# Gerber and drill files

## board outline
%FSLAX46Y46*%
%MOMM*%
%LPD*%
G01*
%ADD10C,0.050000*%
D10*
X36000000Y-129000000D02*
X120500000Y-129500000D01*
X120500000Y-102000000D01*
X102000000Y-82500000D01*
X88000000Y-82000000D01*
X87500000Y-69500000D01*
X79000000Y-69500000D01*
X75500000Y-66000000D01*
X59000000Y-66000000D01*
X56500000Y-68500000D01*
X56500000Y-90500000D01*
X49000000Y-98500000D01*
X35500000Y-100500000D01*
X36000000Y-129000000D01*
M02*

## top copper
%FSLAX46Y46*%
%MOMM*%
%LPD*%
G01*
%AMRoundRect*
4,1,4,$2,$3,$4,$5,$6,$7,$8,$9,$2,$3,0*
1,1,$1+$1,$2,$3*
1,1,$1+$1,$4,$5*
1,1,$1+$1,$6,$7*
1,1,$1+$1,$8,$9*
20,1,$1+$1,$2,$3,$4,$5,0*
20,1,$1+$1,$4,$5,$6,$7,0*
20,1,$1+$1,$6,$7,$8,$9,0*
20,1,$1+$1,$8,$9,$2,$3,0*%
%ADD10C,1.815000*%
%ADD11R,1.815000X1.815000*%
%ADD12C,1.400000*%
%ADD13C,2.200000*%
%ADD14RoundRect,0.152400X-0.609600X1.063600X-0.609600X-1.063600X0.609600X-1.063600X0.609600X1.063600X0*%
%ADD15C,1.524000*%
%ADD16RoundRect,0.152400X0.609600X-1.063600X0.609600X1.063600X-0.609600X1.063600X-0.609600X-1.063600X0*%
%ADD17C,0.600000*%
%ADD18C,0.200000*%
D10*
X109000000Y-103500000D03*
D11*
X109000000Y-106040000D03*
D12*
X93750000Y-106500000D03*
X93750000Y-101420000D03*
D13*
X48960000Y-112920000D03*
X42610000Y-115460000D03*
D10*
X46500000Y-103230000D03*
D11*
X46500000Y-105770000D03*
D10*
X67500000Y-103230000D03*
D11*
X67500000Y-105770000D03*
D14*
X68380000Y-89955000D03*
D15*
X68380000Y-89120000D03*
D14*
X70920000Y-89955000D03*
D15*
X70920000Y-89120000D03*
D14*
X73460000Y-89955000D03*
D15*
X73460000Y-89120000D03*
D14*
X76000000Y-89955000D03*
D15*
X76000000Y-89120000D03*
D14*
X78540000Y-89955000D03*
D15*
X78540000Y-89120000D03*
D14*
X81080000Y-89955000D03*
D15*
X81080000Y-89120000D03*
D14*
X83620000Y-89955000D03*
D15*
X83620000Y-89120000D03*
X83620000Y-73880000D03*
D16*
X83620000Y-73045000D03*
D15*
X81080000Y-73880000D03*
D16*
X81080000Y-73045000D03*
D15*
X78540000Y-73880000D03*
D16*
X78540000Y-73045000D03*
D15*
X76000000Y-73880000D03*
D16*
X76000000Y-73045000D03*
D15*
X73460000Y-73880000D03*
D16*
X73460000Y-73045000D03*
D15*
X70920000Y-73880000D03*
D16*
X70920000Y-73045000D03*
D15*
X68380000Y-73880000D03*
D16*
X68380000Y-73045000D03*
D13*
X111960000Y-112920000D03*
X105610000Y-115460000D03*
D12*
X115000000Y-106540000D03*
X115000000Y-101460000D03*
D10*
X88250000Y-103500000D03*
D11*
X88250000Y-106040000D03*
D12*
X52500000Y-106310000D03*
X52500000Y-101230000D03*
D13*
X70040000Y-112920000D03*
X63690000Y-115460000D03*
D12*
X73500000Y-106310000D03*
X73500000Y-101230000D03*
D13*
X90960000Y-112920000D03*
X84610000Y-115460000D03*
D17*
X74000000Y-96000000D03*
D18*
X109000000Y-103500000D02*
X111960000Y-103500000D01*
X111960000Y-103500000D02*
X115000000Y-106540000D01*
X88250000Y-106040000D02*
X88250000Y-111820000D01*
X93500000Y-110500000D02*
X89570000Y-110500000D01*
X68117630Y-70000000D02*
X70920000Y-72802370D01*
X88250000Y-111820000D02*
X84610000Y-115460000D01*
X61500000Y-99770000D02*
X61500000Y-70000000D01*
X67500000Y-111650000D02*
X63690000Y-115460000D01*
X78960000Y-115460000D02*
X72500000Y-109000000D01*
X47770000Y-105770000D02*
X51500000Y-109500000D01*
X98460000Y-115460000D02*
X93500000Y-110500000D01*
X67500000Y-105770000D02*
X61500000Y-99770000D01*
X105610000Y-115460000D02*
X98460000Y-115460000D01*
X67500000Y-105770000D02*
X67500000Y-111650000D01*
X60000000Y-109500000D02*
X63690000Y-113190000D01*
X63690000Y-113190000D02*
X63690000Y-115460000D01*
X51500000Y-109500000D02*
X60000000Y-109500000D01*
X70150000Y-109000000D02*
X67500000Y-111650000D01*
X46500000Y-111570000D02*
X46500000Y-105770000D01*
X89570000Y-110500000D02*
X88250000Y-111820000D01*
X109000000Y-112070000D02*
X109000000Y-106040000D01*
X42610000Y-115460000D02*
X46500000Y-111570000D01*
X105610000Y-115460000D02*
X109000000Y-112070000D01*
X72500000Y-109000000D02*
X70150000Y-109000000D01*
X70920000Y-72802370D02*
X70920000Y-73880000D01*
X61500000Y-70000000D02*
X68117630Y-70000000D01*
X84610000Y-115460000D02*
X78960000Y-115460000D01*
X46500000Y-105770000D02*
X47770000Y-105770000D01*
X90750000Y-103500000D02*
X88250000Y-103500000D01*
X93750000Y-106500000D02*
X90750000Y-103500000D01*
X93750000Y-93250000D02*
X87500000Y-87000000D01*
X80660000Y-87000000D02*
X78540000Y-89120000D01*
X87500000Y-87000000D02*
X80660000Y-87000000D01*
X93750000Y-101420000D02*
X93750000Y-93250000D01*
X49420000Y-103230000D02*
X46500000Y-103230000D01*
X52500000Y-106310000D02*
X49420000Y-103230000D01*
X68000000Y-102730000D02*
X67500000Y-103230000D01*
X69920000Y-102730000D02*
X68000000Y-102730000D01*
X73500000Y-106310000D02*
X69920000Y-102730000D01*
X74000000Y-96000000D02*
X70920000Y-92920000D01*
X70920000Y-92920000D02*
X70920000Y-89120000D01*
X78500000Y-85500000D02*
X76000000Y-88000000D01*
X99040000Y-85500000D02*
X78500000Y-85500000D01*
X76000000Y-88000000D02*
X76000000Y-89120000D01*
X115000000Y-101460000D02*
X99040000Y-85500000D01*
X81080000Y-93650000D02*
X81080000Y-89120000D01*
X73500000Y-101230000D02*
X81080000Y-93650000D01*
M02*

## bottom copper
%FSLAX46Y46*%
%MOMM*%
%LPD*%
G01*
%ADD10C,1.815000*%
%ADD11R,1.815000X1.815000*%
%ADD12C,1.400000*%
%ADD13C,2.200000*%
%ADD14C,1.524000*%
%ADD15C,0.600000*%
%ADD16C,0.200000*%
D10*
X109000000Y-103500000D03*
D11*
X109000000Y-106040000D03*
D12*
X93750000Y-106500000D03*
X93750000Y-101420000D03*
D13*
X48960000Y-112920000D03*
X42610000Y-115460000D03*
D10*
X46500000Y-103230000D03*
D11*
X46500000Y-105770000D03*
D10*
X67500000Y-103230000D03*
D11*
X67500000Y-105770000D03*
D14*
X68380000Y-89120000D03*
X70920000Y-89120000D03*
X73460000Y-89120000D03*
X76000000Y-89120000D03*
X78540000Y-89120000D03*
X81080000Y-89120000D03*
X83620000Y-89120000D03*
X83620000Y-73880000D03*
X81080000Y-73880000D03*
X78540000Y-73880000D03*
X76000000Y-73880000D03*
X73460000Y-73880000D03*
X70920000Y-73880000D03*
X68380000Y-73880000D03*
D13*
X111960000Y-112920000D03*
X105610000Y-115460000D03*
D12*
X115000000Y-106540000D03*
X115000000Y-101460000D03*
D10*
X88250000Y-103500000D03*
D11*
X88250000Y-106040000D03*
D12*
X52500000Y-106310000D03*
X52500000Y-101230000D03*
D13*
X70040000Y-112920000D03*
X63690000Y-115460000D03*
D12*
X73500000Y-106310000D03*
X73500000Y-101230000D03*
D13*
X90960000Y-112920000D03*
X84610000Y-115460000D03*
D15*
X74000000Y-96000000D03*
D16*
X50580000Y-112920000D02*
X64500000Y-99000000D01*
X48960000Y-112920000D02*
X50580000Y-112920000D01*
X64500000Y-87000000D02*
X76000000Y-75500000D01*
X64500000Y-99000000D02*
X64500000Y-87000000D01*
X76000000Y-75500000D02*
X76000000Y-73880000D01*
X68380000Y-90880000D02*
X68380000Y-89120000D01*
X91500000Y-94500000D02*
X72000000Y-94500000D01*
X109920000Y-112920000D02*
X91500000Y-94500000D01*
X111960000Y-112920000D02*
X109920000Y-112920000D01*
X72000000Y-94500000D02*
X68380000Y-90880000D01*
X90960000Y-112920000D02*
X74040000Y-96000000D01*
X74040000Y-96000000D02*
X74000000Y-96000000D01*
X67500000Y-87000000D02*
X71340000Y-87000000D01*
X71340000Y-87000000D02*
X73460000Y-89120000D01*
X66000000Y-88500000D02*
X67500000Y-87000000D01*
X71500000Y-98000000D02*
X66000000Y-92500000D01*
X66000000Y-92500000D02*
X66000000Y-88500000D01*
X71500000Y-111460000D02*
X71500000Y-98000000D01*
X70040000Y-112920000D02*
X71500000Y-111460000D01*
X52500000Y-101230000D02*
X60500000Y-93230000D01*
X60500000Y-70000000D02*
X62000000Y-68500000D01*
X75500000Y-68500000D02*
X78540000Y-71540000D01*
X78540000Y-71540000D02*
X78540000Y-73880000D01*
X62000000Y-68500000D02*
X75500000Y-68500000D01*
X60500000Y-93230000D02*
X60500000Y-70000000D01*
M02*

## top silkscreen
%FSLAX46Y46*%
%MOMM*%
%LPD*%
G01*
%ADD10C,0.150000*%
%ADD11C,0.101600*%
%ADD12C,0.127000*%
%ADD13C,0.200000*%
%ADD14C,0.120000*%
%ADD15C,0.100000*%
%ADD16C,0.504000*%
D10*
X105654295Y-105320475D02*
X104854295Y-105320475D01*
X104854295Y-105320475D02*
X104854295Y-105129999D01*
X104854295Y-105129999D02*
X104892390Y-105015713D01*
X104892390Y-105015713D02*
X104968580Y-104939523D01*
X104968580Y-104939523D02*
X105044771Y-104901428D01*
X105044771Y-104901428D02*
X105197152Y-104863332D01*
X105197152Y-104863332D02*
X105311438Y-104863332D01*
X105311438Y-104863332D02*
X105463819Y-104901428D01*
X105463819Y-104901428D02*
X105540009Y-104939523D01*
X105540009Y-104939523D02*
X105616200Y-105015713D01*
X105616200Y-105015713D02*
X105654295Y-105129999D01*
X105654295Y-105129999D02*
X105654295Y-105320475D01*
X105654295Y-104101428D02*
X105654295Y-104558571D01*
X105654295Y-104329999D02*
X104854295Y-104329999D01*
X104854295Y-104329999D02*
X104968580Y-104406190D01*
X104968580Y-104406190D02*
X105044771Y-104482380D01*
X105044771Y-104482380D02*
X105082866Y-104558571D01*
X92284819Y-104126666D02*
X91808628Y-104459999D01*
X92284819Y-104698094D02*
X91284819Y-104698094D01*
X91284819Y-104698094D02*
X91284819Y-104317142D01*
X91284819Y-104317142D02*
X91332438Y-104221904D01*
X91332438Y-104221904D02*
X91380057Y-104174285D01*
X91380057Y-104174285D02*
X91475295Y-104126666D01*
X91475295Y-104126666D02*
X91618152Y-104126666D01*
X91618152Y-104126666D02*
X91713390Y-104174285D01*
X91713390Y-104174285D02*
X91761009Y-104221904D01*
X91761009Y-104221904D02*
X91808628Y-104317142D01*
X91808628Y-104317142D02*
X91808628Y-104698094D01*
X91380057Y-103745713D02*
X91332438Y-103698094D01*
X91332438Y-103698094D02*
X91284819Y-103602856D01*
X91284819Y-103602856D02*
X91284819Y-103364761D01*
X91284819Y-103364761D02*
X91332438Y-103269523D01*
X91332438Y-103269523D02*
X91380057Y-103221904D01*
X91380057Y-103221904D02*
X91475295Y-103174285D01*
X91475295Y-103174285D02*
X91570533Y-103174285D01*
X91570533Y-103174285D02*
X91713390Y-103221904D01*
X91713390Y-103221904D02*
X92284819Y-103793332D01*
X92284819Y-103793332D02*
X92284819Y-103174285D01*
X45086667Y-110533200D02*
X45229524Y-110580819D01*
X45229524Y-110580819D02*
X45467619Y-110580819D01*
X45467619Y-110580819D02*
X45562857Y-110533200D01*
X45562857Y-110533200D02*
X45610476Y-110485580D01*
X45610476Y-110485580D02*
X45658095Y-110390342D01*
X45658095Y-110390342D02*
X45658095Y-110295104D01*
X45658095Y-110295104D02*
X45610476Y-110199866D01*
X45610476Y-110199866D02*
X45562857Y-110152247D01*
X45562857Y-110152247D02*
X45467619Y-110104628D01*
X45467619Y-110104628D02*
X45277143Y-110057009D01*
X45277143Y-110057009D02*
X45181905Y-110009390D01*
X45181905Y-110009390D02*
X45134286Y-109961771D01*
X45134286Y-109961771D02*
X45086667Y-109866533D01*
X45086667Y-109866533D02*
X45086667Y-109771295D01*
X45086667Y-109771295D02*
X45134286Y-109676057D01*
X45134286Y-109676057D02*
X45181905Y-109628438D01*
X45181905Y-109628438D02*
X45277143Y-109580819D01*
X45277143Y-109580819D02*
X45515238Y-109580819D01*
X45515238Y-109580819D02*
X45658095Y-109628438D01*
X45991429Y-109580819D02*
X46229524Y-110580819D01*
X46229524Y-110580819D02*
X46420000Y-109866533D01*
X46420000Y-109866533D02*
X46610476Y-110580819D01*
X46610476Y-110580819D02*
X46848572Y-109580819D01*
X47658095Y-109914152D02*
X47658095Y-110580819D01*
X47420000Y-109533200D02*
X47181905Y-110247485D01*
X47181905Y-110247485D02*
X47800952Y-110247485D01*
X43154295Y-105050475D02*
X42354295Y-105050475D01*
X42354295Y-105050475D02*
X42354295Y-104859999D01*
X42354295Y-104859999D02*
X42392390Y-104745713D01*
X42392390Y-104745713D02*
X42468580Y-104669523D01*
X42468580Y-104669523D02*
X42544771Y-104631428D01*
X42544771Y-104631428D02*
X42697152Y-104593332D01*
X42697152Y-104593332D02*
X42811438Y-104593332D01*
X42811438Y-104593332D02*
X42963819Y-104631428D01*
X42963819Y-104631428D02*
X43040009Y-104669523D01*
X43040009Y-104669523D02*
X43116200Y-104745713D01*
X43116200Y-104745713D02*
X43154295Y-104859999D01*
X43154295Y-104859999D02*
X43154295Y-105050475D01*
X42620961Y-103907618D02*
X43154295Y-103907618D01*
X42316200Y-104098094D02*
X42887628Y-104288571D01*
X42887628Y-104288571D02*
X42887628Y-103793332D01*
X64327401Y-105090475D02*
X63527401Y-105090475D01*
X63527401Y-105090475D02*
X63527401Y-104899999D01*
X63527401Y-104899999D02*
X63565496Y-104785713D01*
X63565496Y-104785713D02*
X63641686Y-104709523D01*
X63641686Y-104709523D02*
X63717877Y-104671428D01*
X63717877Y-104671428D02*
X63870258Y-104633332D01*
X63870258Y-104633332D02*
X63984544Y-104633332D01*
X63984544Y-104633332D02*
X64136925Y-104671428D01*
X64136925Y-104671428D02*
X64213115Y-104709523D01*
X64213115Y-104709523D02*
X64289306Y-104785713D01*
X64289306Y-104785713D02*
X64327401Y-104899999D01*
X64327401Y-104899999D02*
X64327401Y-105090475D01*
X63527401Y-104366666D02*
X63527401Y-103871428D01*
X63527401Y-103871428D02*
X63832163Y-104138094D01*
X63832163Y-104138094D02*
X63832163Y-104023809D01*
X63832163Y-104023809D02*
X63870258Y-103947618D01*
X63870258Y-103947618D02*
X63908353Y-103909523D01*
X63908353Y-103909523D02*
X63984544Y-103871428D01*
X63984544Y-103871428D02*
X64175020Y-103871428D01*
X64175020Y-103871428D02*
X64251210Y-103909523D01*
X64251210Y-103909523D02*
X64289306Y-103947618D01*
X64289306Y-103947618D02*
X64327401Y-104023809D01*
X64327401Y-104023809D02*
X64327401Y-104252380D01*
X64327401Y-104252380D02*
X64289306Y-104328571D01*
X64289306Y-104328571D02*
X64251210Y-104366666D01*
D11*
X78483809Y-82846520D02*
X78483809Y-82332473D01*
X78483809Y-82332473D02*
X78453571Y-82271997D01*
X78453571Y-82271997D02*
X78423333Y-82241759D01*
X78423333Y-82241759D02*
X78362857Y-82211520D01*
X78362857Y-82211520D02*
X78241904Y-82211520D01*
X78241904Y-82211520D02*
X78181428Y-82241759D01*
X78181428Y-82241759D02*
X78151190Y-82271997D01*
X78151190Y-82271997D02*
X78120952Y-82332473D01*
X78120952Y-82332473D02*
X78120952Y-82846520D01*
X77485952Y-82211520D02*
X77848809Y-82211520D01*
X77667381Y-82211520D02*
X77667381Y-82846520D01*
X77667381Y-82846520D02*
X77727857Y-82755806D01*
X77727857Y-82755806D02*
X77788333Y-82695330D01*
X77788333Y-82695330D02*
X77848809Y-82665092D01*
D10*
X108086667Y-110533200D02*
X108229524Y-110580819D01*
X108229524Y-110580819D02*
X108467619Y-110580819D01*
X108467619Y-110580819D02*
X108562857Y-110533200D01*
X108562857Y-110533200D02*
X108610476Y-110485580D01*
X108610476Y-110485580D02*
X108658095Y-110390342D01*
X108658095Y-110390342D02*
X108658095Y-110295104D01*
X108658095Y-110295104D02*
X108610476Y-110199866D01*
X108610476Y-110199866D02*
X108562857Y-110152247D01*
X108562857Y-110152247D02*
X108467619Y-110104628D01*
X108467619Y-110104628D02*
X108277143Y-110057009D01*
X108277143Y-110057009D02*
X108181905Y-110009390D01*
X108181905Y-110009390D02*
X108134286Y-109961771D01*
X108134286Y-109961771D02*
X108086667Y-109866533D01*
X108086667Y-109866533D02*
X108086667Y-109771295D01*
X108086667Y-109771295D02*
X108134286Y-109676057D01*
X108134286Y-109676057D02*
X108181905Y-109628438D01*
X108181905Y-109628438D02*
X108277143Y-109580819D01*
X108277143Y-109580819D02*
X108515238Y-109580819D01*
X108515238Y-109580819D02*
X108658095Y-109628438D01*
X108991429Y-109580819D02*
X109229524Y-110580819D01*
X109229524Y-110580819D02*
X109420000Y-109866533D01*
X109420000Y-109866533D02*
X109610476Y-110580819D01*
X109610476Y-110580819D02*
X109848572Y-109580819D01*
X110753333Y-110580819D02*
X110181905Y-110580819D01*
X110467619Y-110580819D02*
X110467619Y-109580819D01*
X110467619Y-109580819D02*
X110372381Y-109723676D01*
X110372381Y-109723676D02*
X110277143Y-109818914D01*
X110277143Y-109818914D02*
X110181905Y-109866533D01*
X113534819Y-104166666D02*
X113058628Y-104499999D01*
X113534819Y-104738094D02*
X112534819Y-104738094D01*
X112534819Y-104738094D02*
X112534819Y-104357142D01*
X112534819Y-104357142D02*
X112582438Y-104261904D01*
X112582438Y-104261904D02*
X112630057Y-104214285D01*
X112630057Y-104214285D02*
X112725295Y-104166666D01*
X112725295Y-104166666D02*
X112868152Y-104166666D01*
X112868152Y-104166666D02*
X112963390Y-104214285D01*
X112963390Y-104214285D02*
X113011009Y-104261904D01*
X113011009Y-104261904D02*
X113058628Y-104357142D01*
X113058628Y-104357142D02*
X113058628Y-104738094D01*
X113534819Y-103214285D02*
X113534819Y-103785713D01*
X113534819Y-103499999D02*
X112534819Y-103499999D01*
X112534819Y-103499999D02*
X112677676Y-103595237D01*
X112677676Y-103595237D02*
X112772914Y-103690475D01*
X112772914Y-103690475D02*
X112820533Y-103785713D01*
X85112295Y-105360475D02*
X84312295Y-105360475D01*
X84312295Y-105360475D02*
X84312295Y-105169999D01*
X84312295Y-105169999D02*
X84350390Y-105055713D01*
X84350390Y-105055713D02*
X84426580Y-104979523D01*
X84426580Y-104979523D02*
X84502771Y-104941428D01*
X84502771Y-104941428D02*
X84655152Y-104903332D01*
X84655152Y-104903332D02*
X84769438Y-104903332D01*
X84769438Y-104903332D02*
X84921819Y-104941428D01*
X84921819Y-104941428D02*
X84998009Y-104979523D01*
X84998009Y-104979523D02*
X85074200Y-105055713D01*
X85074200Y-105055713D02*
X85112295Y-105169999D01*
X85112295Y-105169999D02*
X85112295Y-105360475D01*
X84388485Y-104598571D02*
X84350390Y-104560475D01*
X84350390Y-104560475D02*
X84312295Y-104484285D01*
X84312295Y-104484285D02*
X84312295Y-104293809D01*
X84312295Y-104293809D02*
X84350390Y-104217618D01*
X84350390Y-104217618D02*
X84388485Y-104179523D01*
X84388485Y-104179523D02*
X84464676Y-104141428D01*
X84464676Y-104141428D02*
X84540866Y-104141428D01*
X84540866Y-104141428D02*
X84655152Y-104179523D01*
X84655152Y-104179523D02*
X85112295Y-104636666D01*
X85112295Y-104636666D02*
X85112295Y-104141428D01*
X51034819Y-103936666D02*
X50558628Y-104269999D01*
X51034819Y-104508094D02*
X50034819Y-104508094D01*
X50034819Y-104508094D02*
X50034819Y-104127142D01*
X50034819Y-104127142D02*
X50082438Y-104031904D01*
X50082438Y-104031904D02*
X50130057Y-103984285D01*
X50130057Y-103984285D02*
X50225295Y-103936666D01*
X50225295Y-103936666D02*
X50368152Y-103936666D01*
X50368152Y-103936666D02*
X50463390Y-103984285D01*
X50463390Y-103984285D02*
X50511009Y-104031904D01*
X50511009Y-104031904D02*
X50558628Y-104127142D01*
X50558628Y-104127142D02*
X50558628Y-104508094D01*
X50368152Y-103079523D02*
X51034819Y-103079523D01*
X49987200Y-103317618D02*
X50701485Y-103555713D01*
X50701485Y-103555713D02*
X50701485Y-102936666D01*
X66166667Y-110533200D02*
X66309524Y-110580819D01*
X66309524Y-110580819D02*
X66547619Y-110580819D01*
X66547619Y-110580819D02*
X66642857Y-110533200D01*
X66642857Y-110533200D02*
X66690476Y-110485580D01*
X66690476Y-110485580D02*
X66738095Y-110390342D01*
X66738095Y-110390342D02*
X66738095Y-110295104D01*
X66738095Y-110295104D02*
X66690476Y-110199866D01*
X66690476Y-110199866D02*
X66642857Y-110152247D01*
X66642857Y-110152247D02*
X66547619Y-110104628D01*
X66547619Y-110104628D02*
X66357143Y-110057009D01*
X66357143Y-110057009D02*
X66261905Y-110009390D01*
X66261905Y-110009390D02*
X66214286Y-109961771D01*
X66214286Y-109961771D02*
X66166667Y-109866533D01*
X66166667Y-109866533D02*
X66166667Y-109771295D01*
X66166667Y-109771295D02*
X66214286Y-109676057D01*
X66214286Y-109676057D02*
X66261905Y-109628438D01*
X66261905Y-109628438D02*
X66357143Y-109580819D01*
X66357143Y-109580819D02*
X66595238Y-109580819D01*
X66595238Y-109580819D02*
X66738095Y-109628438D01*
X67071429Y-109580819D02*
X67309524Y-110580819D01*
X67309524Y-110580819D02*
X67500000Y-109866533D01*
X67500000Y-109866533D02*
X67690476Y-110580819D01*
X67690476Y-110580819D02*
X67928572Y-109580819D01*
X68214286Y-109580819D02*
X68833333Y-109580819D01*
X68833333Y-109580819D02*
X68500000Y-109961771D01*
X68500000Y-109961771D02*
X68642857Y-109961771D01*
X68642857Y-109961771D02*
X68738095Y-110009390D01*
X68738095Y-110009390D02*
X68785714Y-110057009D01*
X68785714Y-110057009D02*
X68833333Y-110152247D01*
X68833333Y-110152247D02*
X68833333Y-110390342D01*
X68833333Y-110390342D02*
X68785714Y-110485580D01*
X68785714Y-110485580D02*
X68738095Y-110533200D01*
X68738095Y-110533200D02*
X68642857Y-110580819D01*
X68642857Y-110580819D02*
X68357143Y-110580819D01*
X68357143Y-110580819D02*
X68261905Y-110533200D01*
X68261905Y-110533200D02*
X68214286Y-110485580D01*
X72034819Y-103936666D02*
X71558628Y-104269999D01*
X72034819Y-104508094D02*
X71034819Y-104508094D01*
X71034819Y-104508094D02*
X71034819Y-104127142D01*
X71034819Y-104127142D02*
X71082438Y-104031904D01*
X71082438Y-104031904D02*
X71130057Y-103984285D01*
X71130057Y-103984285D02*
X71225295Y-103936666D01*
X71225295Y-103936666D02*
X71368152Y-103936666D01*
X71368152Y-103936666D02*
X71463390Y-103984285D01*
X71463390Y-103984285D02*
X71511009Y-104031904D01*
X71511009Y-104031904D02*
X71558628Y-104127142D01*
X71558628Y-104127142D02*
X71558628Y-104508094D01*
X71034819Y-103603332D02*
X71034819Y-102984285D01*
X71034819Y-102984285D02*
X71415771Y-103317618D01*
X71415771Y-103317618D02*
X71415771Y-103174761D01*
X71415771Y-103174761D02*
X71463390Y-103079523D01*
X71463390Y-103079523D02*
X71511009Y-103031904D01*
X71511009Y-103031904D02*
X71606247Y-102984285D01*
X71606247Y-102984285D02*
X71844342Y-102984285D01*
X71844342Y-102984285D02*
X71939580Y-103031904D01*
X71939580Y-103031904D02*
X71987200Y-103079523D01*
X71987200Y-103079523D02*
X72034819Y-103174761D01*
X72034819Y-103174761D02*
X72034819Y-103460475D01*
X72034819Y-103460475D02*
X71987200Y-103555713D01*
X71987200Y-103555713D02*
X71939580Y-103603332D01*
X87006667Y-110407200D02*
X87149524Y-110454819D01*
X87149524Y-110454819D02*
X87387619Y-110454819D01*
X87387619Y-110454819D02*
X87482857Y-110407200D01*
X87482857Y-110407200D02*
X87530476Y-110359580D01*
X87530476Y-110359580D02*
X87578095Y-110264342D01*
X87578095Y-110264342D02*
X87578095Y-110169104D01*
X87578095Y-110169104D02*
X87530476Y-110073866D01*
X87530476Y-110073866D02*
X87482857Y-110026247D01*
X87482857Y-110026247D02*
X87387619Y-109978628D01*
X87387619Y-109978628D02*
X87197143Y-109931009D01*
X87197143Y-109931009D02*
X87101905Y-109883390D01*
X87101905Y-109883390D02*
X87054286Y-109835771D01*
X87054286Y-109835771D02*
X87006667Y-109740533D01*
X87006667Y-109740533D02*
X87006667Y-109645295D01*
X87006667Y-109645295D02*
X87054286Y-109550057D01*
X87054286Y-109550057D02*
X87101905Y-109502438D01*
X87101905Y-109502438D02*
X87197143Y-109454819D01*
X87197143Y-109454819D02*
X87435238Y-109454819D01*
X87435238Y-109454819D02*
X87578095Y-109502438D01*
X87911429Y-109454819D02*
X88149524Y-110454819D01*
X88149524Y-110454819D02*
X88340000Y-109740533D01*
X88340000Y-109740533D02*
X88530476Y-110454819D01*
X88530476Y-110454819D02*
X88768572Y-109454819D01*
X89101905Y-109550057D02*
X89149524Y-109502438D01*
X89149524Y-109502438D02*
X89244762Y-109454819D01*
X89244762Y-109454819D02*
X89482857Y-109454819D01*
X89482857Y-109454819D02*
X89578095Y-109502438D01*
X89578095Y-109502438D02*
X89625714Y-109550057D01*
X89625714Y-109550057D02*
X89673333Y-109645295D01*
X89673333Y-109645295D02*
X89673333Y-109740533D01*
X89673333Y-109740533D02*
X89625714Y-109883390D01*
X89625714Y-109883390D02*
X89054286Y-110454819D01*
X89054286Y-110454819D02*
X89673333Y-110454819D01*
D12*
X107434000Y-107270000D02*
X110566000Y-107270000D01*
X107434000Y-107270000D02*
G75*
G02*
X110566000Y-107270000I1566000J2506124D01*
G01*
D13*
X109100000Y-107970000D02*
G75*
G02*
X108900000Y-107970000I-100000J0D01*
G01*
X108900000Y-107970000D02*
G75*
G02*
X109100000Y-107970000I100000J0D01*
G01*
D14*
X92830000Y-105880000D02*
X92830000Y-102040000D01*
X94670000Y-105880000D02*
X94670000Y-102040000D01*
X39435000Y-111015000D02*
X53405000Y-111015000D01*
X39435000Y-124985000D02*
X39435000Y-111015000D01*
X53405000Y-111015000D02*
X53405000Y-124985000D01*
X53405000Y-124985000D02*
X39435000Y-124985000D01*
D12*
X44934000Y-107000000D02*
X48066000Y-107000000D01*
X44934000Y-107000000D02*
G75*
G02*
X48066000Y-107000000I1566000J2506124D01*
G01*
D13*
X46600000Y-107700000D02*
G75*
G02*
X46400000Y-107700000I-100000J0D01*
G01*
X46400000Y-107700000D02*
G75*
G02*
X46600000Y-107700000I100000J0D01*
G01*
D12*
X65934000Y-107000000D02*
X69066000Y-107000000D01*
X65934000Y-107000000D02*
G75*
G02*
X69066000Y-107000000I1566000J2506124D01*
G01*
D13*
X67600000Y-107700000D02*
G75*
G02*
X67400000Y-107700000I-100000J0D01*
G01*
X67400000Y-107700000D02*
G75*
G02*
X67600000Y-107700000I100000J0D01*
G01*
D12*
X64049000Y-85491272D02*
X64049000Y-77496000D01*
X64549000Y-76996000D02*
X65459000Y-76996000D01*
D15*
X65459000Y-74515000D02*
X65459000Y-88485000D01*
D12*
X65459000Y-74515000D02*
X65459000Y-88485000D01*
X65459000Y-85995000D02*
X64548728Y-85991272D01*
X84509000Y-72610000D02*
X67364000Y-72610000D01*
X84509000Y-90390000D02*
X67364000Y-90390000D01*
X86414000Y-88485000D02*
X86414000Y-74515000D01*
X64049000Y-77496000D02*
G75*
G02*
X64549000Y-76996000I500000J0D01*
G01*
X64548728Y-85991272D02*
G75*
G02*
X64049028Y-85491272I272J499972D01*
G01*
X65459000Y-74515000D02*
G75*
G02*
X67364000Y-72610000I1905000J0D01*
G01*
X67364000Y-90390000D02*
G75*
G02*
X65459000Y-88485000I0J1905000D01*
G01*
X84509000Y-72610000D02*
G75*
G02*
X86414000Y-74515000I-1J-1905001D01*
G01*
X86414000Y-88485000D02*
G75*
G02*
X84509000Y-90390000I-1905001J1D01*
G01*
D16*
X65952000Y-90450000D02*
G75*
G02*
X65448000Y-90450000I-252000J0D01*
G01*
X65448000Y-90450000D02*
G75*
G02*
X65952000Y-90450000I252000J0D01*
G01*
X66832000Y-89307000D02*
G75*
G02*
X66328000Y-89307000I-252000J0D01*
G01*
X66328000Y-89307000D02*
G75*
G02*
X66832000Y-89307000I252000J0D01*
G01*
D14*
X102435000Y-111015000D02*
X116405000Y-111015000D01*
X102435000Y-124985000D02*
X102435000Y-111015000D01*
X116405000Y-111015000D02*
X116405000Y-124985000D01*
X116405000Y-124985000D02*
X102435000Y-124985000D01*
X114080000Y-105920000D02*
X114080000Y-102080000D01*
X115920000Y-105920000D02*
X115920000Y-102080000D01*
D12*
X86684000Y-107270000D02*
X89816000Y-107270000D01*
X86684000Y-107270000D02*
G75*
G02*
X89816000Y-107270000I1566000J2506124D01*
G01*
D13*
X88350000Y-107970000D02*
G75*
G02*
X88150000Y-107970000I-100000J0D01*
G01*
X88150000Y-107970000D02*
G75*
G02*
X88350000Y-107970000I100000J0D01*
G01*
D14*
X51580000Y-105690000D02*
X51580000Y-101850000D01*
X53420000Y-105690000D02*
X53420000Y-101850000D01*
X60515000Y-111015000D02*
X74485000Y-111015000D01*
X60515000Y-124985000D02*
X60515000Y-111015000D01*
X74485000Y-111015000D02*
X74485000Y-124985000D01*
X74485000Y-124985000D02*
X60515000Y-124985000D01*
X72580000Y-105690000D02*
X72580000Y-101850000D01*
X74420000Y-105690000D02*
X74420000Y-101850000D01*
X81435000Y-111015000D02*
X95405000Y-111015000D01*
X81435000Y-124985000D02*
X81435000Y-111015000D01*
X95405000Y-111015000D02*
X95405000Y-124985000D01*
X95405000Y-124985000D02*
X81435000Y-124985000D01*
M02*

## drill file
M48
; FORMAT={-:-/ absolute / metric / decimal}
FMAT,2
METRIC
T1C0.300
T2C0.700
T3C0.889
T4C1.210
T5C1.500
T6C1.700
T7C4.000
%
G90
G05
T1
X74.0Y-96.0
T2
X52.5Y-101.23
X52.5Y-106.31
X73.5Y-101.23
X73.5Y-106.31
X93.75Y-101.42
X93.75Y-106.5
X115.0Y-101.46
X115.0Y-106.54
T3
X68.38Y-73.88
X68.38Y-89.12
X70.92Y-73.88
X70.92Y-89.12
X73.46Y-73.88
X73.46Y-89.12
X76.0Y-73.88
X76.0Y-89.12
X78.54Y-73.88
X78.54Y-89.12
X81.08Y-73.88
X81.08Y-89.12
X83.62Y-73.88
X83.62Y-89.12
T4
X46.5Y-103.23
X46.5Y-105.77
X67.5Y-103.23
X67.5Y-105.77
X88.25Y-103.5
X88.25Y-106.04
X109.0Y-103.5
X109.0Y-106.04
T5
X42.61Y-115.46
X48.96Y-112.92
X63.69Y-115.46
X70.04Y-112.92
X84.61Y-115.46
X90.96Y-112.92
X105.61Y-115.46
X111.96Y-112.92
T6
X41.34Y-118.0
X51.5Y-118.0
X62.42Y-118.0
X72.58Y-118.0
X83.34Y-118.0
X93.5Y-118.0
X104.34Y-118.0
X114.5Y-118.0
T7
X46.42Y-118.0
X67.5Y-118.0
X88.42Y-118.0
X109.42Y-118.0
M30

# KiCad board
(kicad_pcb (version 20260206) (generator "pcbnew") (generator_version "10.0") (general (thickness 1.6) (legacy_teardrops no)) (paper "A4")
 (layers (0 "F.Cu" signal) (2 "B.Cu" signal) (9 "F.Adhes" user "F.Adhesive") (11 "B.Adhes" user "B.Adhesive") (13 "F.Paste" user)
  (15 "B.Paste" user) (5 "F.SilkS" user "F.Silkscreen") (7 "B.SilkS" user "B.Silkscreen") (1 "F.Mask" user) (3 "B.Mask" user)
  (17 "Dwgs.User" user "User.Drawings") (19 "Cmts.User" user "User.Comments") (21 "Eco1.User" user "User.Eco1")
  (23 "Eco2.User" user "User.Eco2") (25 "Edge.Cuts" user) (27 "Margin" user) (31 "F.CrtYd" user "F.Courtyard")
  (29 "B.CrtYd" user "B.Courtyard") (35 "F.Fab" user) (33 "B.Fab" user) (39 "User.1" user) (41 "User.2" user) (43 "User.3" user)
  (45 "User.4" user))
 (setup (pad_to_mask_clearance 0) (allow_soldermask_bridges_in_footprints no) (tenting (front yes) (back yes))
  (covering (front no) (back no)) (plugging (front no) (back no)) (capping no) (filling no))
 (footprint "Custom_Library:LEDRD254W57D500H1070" (layer "F.Cu") (at 109 104.77 90)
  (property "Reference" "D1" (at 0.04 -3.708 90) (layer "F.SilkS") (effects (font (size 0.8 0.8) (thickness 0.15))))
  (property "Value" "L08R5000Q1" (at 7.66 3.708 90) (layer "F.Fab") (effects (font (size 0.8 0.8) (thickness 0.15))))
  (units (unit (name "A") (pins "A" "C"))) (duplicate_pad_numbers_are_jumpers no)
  (fp_line (start -2.5 -1.566) (end -2.5 1.566) (stroke (width 0.127) (type solid)) (layer "F.SilkS"))
  (fp_arc (start -2.5 -1.566) (mid 2.961291 0) (end -2.5 1.566) (stroke (width 0.127) (type solid)) (layer "F.SilkS"))
  (fp_circle (center -3.2 0) (end -3.1 0) (stroke (width 0.2) (type solid)) (fill no) (layer "F.SilkS"))
  (pad "A" thru_hole circle (at 1.27 0 90) (size 1.815 1.815) (drill 1.21) (layers "*.Cu" "*.Mask") (remove_unused_layers no)
   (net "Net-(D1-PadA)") (solder_mask_margin 0.102))
  (pad "C" thru_hole rect (at -1.27 0 90) (size 1.815 1.815) (drill 1.21) (layers "*.Cu" "*.Mask") (remove_unused_layers no) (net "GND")
   (solder_mask_margin 0.102)))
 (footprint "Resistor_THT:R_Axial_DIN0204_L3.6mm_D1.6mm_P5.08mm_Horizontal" (layer "F.Cu") (at 93.75 106.5 90)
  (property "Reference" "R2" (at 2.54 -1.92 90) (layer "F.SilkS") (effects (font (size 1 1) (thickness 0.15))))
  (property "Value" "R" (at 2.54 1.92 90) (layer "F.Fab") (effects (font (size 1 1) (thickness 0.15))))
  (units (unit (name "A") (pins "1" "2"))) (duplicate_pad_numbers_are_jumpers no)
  (fp_line (start 0.62 -0.92) (end 4.46 -0.92) (stroke (width 0.12) (type solid)) (layer "F.SilkS"))
  (fp_line (start 0.62 0.92) (end 4.46 0.92) (stroke (width 0.12) (type solid)) (layer "F.SilkS"))
  (pad "1" thru_hole circle (at 0 0 90) (size 1.4 1.4) (drill 0.7) (layers "*.Cu" "*.Mask") (remove_unused_layers no) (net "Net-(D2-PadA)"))
  (pad "2" thru_hole circle (at 5.08 0 90) (size 1.4 1.4) (drill 0.7) (layers "*.Cu" "*.Mask") (remove_unused_layers no) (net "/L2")))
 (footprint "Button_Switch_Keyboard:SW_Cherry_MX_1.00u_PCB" (layer "F.Cu") (at 48.96 112.92)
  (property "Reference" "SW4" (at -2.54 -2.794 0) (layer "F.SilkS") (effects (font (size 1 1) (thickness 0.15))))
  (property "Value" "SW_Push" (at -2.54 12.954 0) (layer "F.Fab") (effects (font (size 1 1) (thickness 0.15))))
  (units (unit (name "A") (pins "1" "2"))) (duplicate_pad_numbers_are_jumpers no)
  (fp_line (start -9.525 -1.905) (end 4.445 -1.905) (stroke (width 0.12) (type solid)) (layer "F.SilkS"))
  (fp_line (start -9.525 12.065) (end -9.525 -1.905) (stroke (width 0.12) (type solid)) (layer "F.SilkS"))
  (fp_line (start 4.445 -1.905) (end 4.445 12.065) (stroke (width 0.12) (type solid)) (layer "F.SilkS"))
  (fp_line (start 4.445 12.065) (end -9.525 12.065) (stroke (width 0.12) (type solid)) (layer "F.SilkS"))
  (pad "" np_thru_hole circle (at -7.62 5.08) (size 1.7 1.7) (drill 1.7) (layers "*.Cu" "*.Mask"))
  (pad "" np_thru_hole circle (at -2.54 5.08) (size 4 4) (drill 4) (layers "*.Cu" "*.Mask"))
  (pad "" np_thru_hole circle (at 2.54 5.08) (size 1.7 1.7) (drill 1.7) (layers "*.Cu" "*.Mask"))
  (pad "1" thru_hole circle (at 0 0) (size 2.2 2.2) (drill 1.5) (layers "*.Cu" "*.Mask") (remove_unused_layers no) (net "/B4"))
  (pad "2" thru_hole circle (at -6.35 2.54) (size 2.2 2.2) (drill 1.5) (layers "*.Cu" "*.Mask") (remove_unused_layers no) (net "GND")))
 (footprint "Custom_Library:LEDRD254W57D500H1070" (layer "F.Cu") (at 46.5 104.5 90)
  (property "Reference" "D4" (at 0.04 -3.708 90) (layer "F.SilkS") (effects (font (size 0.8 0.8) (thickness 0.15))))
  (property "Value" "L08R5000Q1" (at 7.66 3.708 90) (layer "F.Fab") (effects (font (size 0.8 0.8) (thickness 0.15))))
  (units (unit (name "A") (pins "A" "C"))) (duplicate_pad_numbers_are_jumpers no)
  (fp_line (start -2.5 -1.566) (end -2.5 1.566) (stroke (width 0.127) (type solid)) (layer "F.SilkS"))
  (fp_arc (start -2.5 -1.566) (mid 2.961291 0) (end -2.5 1.566) (stroke (width 0.127) (type solid)) (layer "F.SilkS"))
  (fp_circle (center -3.2 0) (end -3.1 0) (stroke (width 0.2) (type solid)) (fill no) (layer "F.SilkS"))
  (pad "A" thru_hole circle (at 1.27 0 90) (size 1.815 1.815) (drill 1.21) (layers "*.Cu" "*.Mask") (remove_unused_layers no)
   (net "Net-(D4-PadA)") (solder_mask_margin 0.102))
  (pad "C" thru_hole rect (at -1.27 0 90) (size 1.815 1.815) (drill 1.21) (layers "*.Cu" "*.Mask") (remove_unused_layers no) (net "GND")
   (solder_mask_margin 0.102)))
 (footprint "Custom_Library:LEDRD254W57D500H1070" (layer "F.Cu") (at 67.5 104.5 90)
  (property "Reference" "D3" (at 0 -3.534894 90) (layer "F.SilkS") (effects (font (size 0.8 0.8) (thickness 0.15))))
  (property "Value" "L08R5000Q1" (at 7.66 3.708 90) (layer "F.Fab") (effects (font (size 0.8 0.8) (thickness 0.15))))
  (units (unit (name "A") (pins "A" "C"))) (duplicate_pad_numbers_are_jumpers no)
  (fp_line (start -2.5 -1.566) (end -2.5 1.566) (stroke (width 0.127) (type solid)) (layer "F.SilkS"))
  (fp_arc (start -2.5 -1.566) (mid 2.961291 0) (end -2.5 1.566) (stroke (width 0.127) (type solid)) (layer "F.SilkS"))
  (fp_circle (center -3.2 0) (end -3.1 0) (stroke (width 0.2) (type solid)) (fill no) (layer "F.SilkS"))
  (pad "A" thru_hole circle (at 1.27 0 90) (size 1.815 1.815) (drill 1.21) (layers "*.Cu" "*.Mask") (remove_unused_layers no)
   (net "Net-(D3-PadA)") (solder_mask_margin 0.102))
  (pad "C" thru_hole rect (at -1.27 0 90) (size 1.815 1.815) (drill 1.21) (layers "*.Cu" "*.Mask") (remove_unused_layers no) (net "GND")
   (solder_mask_margin 0.102)))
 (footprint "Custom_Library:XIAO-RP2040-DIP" (layer "F.Cu") (at 76 81.5 180)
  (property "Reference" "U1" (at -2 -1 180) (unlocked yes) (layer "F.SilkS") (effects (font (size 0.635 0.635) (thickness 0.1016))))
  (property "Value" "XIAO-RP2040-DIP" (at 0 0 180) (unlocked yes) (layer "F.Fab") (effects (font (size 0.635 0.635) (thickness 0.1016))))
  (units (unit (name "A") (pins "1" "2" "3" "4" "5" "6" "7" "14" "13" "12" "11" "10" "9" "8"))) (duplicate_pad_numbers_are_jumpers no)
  (fp_line (start 11.951 -3.991272) (end 11.951 4.004) (stroke (width 0.127) (type solid)) (layer "F.SilkS"))
  (fp_line (start 11.451 4.504) (end 10.541 4.504) (stroke (width 0.127) (type solid)) (layer "F.SilkS"))
  (fp_line (start 10.541 6.985) (end 10.541 -6.985) (stroke (width 0.1) (type solid)) (layer "F.SilkS"))
  (fp_line (start 10.541 6.985) (end 10.541 -6.985) (stroke (width 0.127) (type solid)) (layer "F.SilkS"))
  (fp_line (start 10.541 -4.495) (end 11.451272 -4.491272) (stroke (width 0.127) (type solid)) (layer "F.SilkS"))
  (fp_line (start -8.509 8.89) (end 8.636 8.89) (stroke (width 0.127) (type solid)) (layer "F.SilkS"))
  (fp_line (start -8.509 -8.89) (end 8.636 -8.89) (stroke (width 0.127) (type solid)) (layer "F.SilkS"))
  (fp_line (start -10.414 -6.985) (end -10.414 6.985) (stroke (width 0.127) (type solid)) (layer "F.SilkS"))
  (fp_arc (start 11.951 4.004) (mid 11.804553 4.357553) (end 11.451 4.504) (stroke (width 0.127) (type default)) (layer "F.SilkS"))
  (fp_arc (start 11.451272 -4.491272) (mid 11.804644 -4.344724) (end 11.951 -3.991272) (stroke (width 0.127) (type default))
   (layer "F.SilkS"))
  (fp_arc (start 10.541 6.985) (mid 9.983038 8.332038) (end 8.636 8.89) (stroke (width 0.127) (type solid)) (layer "F.SilkS"))
  (fp_arc (start 8.636 -8.89) (mid 9.983038 -8.332038) (end 10.541 -6.985) (stroke (width 0.127) (type solid)) (layer "F.SilkS"))
  (fp_arc (start -8.509 8.89) (mid -9.856038 8.332038) (end -10.414 6.985) (stroke (width 0.127) (type solid)) (layer "F.SilkS"))
  (fp_arc (start -10.414 -6.985) (mid -9.856038 -8.332038) (end -8.509 -8.89) (stroke (width 0.127) (type solid)) (layer "F.SilkS"))
  (fp_circle (center 10.3 -8.95) (end 10.554 -8.95) (stroke (width 0.5) (type solid)) (fill yes) (layer "F.SilkS"))
  (fp_circle (center 9.42 -7.807) (end 9.674 -7.807) (stroke (width 0.5) (type solid)) (fill yes) (layer "F.SilkS"))
  (pad "1" smd roundrect (at 7.62 -8.455 270) (size 2.432 1.524) (layers "F.Cu" "F.Mask") (roundrect_rratio 0.1) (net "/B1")
   (thermal_bridge_angle 45))
  (pad "1" thru_hole circle (at 7.62 -7.62 270) (size 1.524 1.524) (drill 0.889) (layers "*.Cu" "*.Mask") (remove_unused_layers no)
   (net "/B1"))
  (pad "2" smd roundrect (at 5.08 -8.455 270) (size 2.432 1.524) (layers "F.Cu" "F.Mask") (roundrect_rratio 0.1) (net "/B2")
   (thermal_bridge_angle 45))
  (pad "2" thru_hole circle (at 5.08 -7.62 270) (size 1.524 1.524) (drill 0.889) (layers "*.Cu" "*.Mask") (remove_unused_layers no)
   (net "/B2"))
  (pad "3" smd roundrect (at 2.54 -8.455 270) (size 2.432 1.524) (layers "F.Cu" "F.Mask") (roundrect_rratio 0.1) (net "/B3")
   (thermal_bridge_angle 45))
  (pad "3" thru_hole circle (at 2.54 -7.62 270) (size 1.524 1.524) (drill 0.889) (layers "*.Cu" "*.Mask") (remove_unused_layers no)
   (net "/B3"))
  (pad "4" smd roundrect (at 0 -8.455 270) (size 2.432 1.524) (layers "F.Cu" "F.Mask") (roundrect_rratio 0.1) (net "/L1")
   (thermal_bridge_angle 45))
  (pad "4" thru_hole circle (at 0 -7.62 270) (size 1.524 1.524) (drill 0.889) (layers "*.Cu" "*.Mask") (remove_unused_layers no) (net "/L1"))
  (pad "5" smd roundrect (at -2.54 -8.455 270) (size 2.432 1.524) (layers "F.Cu" "F.Mask") (roundrect_rratio 0.1) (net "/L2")
   (thermal_bridge_angle 45))
  (pad "5" thru_hole circle (at -2.54 -7.62 270) (size 1.524 1.524) (drill 0.889) (layers "*.Cu" "*.Mask") (remove_unused_layers no)
   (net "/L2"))
  (pad "6" smd roundrect (at -5.08 -8.455 270) (size 2.432 1.524) (layers "F.Cu" "F.Mask") (roundrect_rratio 0.1) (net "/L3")
   (thermal_bridge_angle 45))
  (pad "6" thru_hole circle (at -5.08 -7.62 270) (size 1.524 1.524) (drill 0.889) (layers "*.Cu" "*.Mask") (remove_unused_layers no)
   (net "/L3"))
  (pad "7" smd roundrect (at -7.62 -8.455 270) (size 2.432 1.524) (layers "F.Cu" "F.Mask") (roundrect_rratio 0.1)
   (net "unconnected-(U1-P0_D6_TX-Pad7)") (thermal_bridge_angle 45))
  (pad "7" thru_hole circle (at -7.62 -7.62 270) (size 1.524 1.524) (drill 0.889) (layers "*.Cu" "*.Mask") (remove_unused_layers no)
   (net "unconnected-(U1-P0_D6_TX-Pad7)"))
  (pad "8" thru_hole circle (at -7.62 7.62 90) (size 1.524 1.524) (drill 0.889) (layers "*.Cu" "*.Mask") (remove_unused_layers no)
   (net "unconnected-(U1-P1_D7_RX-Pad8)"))
  (pad "8" smd roundrect (at -7.62 8.455 90) (size 2.432 1.524) (layers "F.Cu" "F.Mask") (roundrect_rratio 0.1)
   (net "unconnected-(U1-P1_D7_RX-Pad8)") (thermal_bridge_angle 45))
  (pad "9" thru_hole circle (at -5.08 7.62 90) (size 1.524 1.524) (drill 0.889) (layers "*.Cu" "*.Mask") (remove_unused_layers no)
   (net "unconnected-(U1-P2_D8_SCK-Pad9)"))
  (pad "9" smd roundrect (at -5.08 8.455 90) (size 2.432 1.524) (layers "F.Cu" "F.Mask") (roundrect_rratio 0.1)
   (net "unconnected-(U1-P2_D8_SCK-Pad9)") (thermal_bridge_angle 45))
  (pad "10" thru_hole circle (at -2.54 7.62 90) (size 1.524 1.524) (drill 0.889) (layers "*.Cu" "*.Mask") (remove_unused_layers no)
   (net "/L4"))
  (pad "10" smd roundrect (at -2.54 8.455 90) (size 2.432 1.524) (layers "F.Cu" "F.Mask") (roundrect_rratio 0.1) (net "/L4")
   (thermal_bridge_angle 45))
  (pad "11" thru_hole circle (at 0 7.62 90) (size 1.524 1.524) (drill 0.889) (layers "*.Cu" "*.Mask") (remove_unused_layers no) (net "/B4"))
  (pad "11" smd roundrect (at 0 8.455 90) (size 2.432 1.524) (layers "F.Cu" "F.Mask") (roundrect_rratio 0.1) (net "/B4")
   (thermal_bridge_angle 45))
  (pad "12" thru_hole circle (at 2.54 7.62 90) (size 1.524 1.524) (drill 0.889) (layers "*.Cu" "*.Mask") (remove_unused_layers no)
   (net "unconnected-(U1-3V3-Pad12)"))
  (pad "12" smd roundrect (at 2.54 8.455 90) (size 2.432 1.524) (layers "F.Cu" "F.Mask") (roundrect_rratio 0.1)
   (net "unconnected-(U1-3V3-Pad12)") (thermal_bridge_angle 45))
  (pad "13" thru_hole circle (at 5.08 7.62 90) (size 1.524 1.524) (drill 0.889) (layers "*.Cu" "*.Mask") (remove_unused_layers no)
   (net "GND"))
  (pad "13" smd roundrect (at 5.08 8.455 90) (size 2.432 1.524) (layers "F.Cu" "F.Mask") (roundrect_rratio 0.1) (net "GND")
   (thermal_bridge_angle 45))
  (pad "14" thru_hole circle (at 7.62 7.62 90) (size 1.524 1.524) (drill 0.889) (layers "*.Cu" "*.Mask") (remove_unused_layers no)
   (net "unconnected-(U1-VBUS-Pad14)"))
  (pad "14" smd roundrect (at 7.62 8.455 90) (size 2.432 1.524) (layers "F.Cu" "F.Mask") (roundrect_rratio 0.1)
   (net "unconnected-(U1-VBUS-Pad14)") (thermal_bridge_angle 45)))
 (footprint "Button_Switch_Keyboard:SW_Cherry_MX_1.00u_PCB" (layer "F.Cu") (at 111.96 112.92)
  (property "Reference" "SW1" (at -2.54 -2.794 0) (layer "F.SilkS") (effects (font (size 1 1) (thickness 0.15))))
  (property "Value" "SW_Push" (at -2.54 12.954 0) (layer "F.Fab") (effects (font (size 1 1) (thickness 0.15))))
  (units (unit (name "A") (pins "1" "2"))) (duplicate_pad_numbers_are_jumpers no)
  (fp_line (start -9.525 -1.905) (end 4.445 -1.905) (stroke (width 0.12) (type solid)) (layer "F.SilkS"))
  (fp_line (start -9.525 12.065) (end -9.525 -1.905) (stroke (width 0.12) (type solid)) (layer "F.SilkS"))
  (fp_line (start 4.445 -1.905) (end 4.445 12.065) (stroke (width 0.12) (type solid)) (layer "F.SilkS"))
  (fp_line (start 4.445 12.065) (end -9.525 12.065) (stroke (width 0.12) (type solid)) (layer "F.SilkS"))
  (pad "" np_thru_hole circle (at -7.62 5.08) (size 1.7 1.7) (drill 1.7) (layers "*.Cu" "*.Mask"))
  (pad "" np_thru_hole circle (at -2.54 5.08) (size 4 4) (drill 4) (layers "*.Cu" "*.Mask"))
  (pad "" np_thru_hole circle (at 2.54 5.08) (size 1.7 1.7) (drill 1.7) (layers "*.Cu" "*.Mask"))
  (pad "1" thru_hole circle (at 0 0) (size 2.2 2.2) (drill 1.5) (layers "*.Cu" "*.Mask") (remove_unused_layers no) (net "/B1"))
  (pad "2" thru_hole circle (at -6.35 2.54) (size 2.2 2.2) (drill 1.5) (layers "*.Cu" "*.Mask") (remove_unused_layers no) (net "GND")))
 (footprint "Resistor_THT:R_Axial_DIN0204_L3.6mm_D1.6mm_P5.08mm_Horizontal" (layer "F.Cu") (at 115 106.54 90)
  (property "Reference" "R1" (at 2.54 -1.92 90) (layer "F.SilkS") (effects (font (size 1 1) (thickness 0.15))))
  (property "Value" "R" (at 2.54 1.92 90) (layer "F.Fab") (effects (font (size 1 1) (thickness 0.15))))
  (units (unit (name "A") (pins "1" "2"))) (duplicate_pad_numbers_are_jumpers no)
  (fp_line (start 0.62 -0.92) (end 4.46 -0.92) (stroke (width 0.12) (type solid)) (layer "F.SilkS"))
  (fp_line (start 0.62 0.92) (end 4.46 0.92) (stroke (width 0.12) (type solid)) (layer "F.SilkS"))
  (pad "1" thru_hole circle (at 0 0 90) (size 1.4 1.4) (drill 0.7) (layers "*.Cu" "*.Mask") (remove_unused_layers no) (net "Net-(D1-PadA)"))
  (pad "2" thru_hole circle (at 5.08 0 90) (size 1.4 1.4) (drill 0.7) (layers "*.Cu" "*.Mask") (remove_unused_layers no) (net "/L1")))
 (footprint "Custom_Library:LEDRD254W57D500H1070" (layer "F.Cu") (at 88.25 104.77 90)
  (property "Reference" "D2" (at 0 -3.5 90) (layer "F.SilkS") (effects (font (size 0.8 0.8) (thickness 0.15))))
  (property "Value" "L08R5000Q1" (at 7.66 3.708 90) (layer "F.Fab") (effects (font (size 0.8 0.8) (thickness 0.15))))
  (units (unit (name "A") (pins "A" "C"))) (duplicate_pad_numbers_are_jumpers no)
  (fp_line (start -2.5 -1.566) (end -2.5 1.566) (stroke (width 0.127) (type solid)) (layer "F.SilkS"))
  (fp_arc (start -2.5 -1.566) (mid 2.961291 0) (end -2.5 1.566) (stroke (width 0.127) (type solid)) (layer "F.SilkS"))
  (fp_circle (center -3.2 0) (end -3.1 0) (stroke (width 0.2) (type solid)) (fill no) (layer "F.SilkS"))
  (pad "A" thru_hole circle (at 1.27 0 90) (size 1.815 1.815) (drill 1.21) (layers "*.Cu" "*.Mask") (remove_unused_layers no)
   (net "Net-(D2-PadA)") (solder_mask_margin 0.102))
  (pad "C" thru_hole rect (at -1.27 0 90) (size 1.815 1.815) (drill 1.21) (layers "*.Cu" "*.Mask") (remove_unused_layers no) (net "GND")
   (solder_mask_margin 0.102)))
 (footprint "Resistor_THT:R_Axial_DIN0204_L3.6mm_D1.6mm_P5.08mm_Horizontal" (layer "F.Cu") (at 52.5 106.31 90)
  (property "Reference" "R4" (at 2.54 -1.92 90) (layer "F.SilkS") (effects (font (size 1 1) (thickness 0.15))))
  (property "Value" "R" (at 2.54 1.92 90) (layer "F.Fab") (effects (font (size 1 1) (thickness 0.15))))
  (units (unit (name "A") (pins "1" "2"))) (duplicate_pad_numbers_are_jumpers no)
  (fp_line (start 0.62 -0.92) (end 4.46 -0.92) (stroke (width 0.12) (type solid)) (layer "F.SilkS"))
  (fp_line (start 0.62 0.92) (end 4.46 0.92) (stroke (width 0.12) (type solid)) (layer "F.SilkS"))
  (pad "1" thru_hole circle (at 0 0 90) (size 1.4 1.4) (drill 0.7) (layers "*.Cu" "*.Mask") (remove_unused_layers no) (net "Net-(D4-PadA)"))
  (pad "2" thru_hole circle (at 5.08 0 90) (size 1.4 1.4) (drill 0.7) (layers "*.Cu" "*.Mask") (remove_unused_layers no) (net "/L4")))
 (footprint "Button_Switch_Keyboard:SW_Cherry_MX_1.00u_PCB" (layer "F.Cu") (at 70.04 112.92)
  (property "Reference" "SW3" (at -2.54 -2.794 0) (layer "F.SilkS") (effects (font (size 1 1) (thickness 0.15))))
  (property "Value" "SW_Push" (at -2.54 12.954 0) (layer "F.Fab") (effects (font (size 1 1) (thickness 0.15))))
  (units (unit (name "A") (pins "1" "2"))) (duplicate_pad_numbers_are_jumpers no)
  (fp_line (start -9.525 -1.905) (end 4.445 -1.905) (stroke (width 0.12) (type solid)) (layer "F.SilkS"))
  (fp_line (start -9.525 12.065) (end -9.525 -1.905) (stroke (width 0.12) (type solid)) (layer "F.SilkS"))
  (fp_line (start 4.445 -1.905) (end 4.445 12.065) (stroke (width 0.12) (type solid)) (layer "F.SilkS"))
  (fp_line (start 4.445 12.065) (end -9.525 12.065) (stroke (width 0.12) (type solid)) (layer "F.SilkS"))
  (pad "" np_thru_hole circle (at -7.62 5.08) (size 1.7 1.7) (drill 1.7) (layers "*.Cu" "*.Mask"))
  (pad "" np_thru_hole circle (at -2.54 5.08) (size 4 4) (drill 4) (layers "*.Cu" "*.Mask"))
  (pad "" np_thru_hole circle (at 2.54 5.08) (size 1.7 1.7) (drill 1.7) (layers "*.Cu" "*.Mask"))
  (pad "1" thru_hole circle (at 0 0) (size 2.2 2.2) (drill 1.5) (layers "*.Cu" "*.Mask") (remove_unused_layers no) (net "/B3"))
  (pad "2" thru_hole circle (at -6.35 2.54) (size 2.2 2.2) (drill 1.5) (layers "*.Cu" "*.Mask") (remove_unused_layers no) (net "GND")))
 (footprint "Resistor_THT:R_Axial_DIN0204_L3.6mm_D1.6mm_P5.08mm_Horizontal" (layer "F.Cu") (at 73.5 106.31 90)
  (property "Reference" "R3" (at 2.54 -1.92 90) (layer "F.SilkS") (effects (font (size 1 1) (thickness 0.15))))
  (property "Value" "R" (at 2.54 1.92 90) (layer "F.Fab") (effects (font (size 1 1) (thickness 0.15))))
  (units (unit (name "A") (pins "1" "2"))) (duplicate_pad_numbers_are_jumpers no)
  (fp_line (start 0.62 -0.92) (end 4.46 -0.92) (stroke (width 0.12) (type solid)) (layer "F.SilkS"))
  (fp_line (start 0.62 0.92) (end 4.46 0.92) (stroke (width 0.12) (type solid)) (layer "F.SilkS"))
  (pad "1" thru_hole circle (at 0 0 90) (size 1.4 1.4) (drill 0.7) (layers "*.Cu" "*.Mask") (remove_unused_layers no) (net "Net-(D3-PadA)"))
  (pad "2" thru_hole circle (at 5.08 0 90) (size 1.4 1.4) (drill 0.7) (layers "*.Cu" "*.Mask") (remove_unused_layers no) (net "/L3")))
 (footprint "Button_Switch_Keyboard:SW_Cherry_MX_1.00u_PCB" (layer "F.Cu") (at 90.96 112.92)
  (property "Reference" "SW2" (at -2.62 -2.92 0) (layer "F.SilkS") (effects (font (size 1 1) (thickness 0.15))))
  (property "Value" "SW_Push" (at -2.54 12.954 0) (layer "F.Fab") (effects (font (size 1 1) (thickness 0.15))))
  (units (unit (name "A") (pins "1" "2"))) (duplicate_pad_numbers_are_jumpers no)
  (fp_line (start -9.525 -1.905) (end 4.445 -1.905) (stroke (width 0.12) (type solid)) (layer "F.SilkS"))
  (fp_line (start -9.525 12.065) (end -9.525 -1.905) (stroke (width 0.12) (type solid)) (layer "F.SilkS"))
  (fp_line (start 4.445 -1.905) (end 4.445 12.065) (stroke (width 0.12) (type solid)) (layer "F.SilkS"))
  (fp_line (start 4.445 12.065) (end -9.525 12.065) (stroke (width 0.12) (type solid)) (layer "F.SilkS"))
  (pad "" np_thru_hole circle (at -7.62 5.08) (size 1.7 1.7) (drill 1.7) (layers "*.Cu" "*.Mask"))
  (pad "" np_thru_hole circle (at -2.54 5.08) (size 4 4) (drill 4) (layers "*.Cu" "*.Mask"))
  (pad "" np_thru_hole circle (at 2.54 5.08) (size 1.7 1.7) (drill 1.7) (layers "*.Cu" "*.Mask"))
  (pad "1" thru_hole circle (at 0 0) (size 2.2 2.2) (drill 1.5) (layers "*.Cu" "*.Mask") (remove_unused_layers no) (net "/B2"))
  (pad "2" thru_hole circle (at -6.35 2.54) (size 2.2 2.2) (drill 1.5) (layers "*.Cu" "*.Mask") (remove_unused_layers no) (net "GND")))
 (gr_poly
  (pts (xy 36 129) (xy 120.5 129.5) (xy 120.5 102) (xy 102 82.5) (xy 88 82) (xy 87.5 69.5) (xy 79 69.5) (xy 75.5 66) (xy 59 66)
   (xy 56.5 68.5) (xy 56.5 90.5) (xy 49 98.5) (xy 35.5 100.5))
  (stroke (width 0.05) (type solid)) (fill no) (locked yes) (layer "Edge.Cuts"))
 (segment (start 109 103.5) (end 111.96 103.5) (width 0.2) (layer "F.Cu") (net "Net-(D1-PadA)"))
 (segment (start 111.96 103.5) (end 115 106.54) (width 0.2) (layer "F.Cu") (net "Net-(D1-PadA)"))
 (segment (start 88.25 106.04) (end 88.25 111.82) (width 0.2) (layer "F.Cu") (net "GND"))
 (segment (start 93.5 110.5) (end 89.57 110.5) (width 0.2) (layer "F.Cu") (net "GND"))
 (segment (start 68.11763 70) (end 70.92 72.80237) (width 0.2) (layer "F.Cu") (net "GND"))
 (segment (start 88.25 111.82) (end 84.61 115.46) (width 0.2) (layer "F.Cu") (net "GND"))
 (segment (start 61.5 99.77) (end 61.5 70) (width 0.2) (layer "F.Cu") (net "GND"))
 (segment (start 67.5 111.65) (end 63.69 115.46) (width 0.2) (layer "F.Cu") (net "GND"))
 (segment (start 78.96 115.46) (end 72.5 109) (width 0.2) (layer "F.Cu") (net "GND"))
 (segment (start 47.77 105.77) (end 51.5 109.5) (width 0.2) (layer "F.Cu") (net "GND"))
 (segment (start 98.46 115.46) (end 93.5 110.5) (width 0.2) (layer "F.Cu") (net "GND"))
 (segment (start 67.5 105.77) (end 61.5 99.77) (width 0.2) (layer "F.Cu") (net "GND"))
 (segment (start 105.61 115.46) (end 98.46 115.46) (width 0.2) (layer "F.Cu") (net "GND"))
 (segment (start 67.5 105.77) (end 67.5 111.65) (width 0.2) (layer "F.Cu") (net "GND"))
 (segment (start 60 109.5) (end 63.69 113.19) (width 0.2) (layer "F.Cu") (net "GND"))
 (segment (start 63.69 113.19) (end 63.69 115.46) (width 0.2) (layer "F.Cu") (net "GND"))
 (segment (start 51.5 109.5) (end 60 109.5) (width 0.2) (layer "F.Cu") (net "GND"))
 (segment (start 70.15 109) (end 67.5 111.65) (width 0.2) (layer "F.Cu") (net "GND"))
 (segment (start 46.5 111.57) (end 46.5 105.77) (width 0.2) (layer "F.Cu") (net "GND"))
 (segment (start 89.57 110.5) (end 88.25 111.82) (width 0.2) (layer "F.Cu") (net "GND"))
 (segment (start 109 112.07) (end 109 106.04) (width 0.2) (layer "F.Cu") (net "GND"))
 (segment (start 42.61 115.46) (end 46.5 111.57) (width 0.2) (layer "F.Cu") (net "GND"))
 (segment (start 105.61 115.46) (end 109 112.07) (width 0.2) (layer "F.Cu") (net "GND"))
 (segment (start 72.5 109) (end 70.15 109) (width 0.2) (layer "F.Cu") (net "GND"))
 (segment (start 70.92 72.80237) (end 70.92 73.88) (width 0.2) (layer "F.Cu") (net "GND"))
 (segment (start 61.5 70) (end 68.11763 70) (width 0.2) (layer "F.Cu") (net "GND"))
 (segment (start 84.61 115.46) (end 78.96 115.46) (width 0.2) (layer "F.Cu") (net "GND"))
 (segment (start 46.5 105.77) (end 47.77 105.77) (width 0.2) (layer "F.Cu") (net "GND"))
 (segment (start 90.75 103.5) (end 88.25 103.5) (width 0.2) (layer "F.Cu") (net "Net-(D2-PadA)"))
 (segment (start 93.75 106.5) (end 90.75 103.5) (width 0.2) (layer "F.Cu") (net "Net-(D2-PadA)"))
 (segment (start 93.75 93.25) (end 87.5 87) (width 0.2) (layer "F.Cu") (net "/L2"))
 (segment (start 80.66 87) (end 78.54 89.12) (width 0.2) (layer "F.Cu") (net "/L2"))
 (segment (start 87.5 87) (end 80.66 87) (width 0.2) (layer "F.Cu") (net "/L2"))
 (segment (start 93.75 101.42) (end 93.75 93.25) (width 0.2) (layer "F.Cu") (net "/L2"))
 (segment (start 50.58 112.92) (end 64.5 99) (width 0.2) (layer "B.Cu") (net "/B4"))
 (segment (start 48.96 112.92) (end 50.58 112.92) (width 0.2) (layer "B.Cu") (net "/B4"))
 (segment (start 64.5 87) (end 76 75.5) (width 0.2) (layer "B.Cu") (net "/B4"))
 (segment (start 64.5 99) (end 64.5 87) (width 0.2) (layer "B.Cu") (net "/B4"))
 (segment (start 76 75.5) (end 76 73.88) (width 0.2) (layer "B.Cu") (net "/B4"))
 (segment (start 49.42 103.23) (end 46.5 103.23) (width 0.2) (layer "F.Cu") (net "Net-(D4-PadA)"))
 (segment (start 52.5 106.31) (end 49.42 103.23) (width 0.2) (layer "F.Cu") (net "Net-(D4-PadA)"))
 (segment (start 68 102.73) (end 67.5 103.23) (width 0.2) (layer "F.Cu") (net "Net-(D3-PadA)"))
 (segment (start 69.92 102.73) (end 68 102.73) (width 0.2) (layer "F.Cu") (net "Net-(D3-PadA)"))
 (segment (start 73.5 106.31) (end 69.92 102.73) (width 0.2) (layer "F.Cu") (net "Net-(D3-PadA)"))
 (segment (start 68.38 90.88) (end 68.38 89.12) (width 0.2) (layer "B.Cu") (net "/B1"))
 (segment (start 91.5 94.5) (end 72 94.5) (width 0.2) (layer "B.Cu") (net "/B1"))
 (segment (start 109.92 112.92) (end 91.5 94.5) (width 0.2) (layer "B.Cu") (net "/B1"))
 (segment (start 111.96 112.92) (end 109.92 112.92) (width 0.2) (layer "B.Cu") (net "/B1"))
 (segment (start 72 94.5) (end 68.38 90.88) (width 0.2) (layer "B.Cu") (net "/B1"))
 (segment (start 74 96) (end 70.92 92.92) (width 0.2) (layer "F.Cu") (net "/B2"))
 (segment (start 70.92 92.92) (end 70.92 89.12) (width 0.2) (layer "F.Cu") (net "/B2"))
 (via (at 74 96) (size 0.6) (drill 0.3) (layers "F.Cu" "B.Cu") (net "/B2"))
 (segment (start 90.96 112.92) (end 74.04 96) (width 0.2) (layer "B.Cu") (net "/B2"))
 (segment (start 74.04 96) (end 74 96) (width 0.2) (layer "B.Cu") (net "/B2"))
 (segment (start 67.5 87) (end 71.34 87) (width 0.2) (layer "B.Cu") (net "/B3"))
 (segment (start 71.34 87) (end 73.46 89.12) (width 0.2) (layer "B.Cu") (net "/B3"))
 (segment (start 66 88.5) (end 67.5 87) (width 0.2) (layer "B.Cu") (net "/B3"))
 (segment (start 71.5 98) (end 66 92.5) (width 0.2) (layer "B.Cu") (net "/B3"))
 (segment (start 66 92.5) (end 66 88.5) (width 0.2) (layer "B.Cu") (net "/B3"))
 (segment (start 71.5 111.46) (end 71.5 98) (width 0.2) (layer "B.Cu") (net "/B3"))
 (segment (start 70.04 112.92) (end 71.5 111.46) (width 0.2) (layer "B.Cu") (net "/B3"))
 (segment (start 78.5 85.5) (end 76 88) (width 0.2) (layer "F.Cu") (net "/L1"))
 (segment (start 99.04 85.5) (end 78.5 85.5) (width 0.2) (layer "F.Cu") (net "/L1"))
 (segment (start 76 88) (end 76 89.12) (width 0.2) (layer "F.Cu") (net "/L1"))
 (segment (start 115 101.46) (end 99.04 85.5) (width 0.2) (layer "F.Cu") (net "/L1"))
 (segment (start 81.08 93.65) (end 81.08 89.12) (width 0.2) (layer "F.Cu") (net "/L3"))
 (segment (start 73.5 101.23) (end 81.08 93.65) (width 0.2) (layer "F.Cu") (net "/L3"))
 (segment (start 52.5 101.23) (end 60.5 93.23) (width 0.2) (layer "B.Cu") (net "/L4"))
 (segment (start 60.5 70) (end 62 68.5) (width 0.2) (layer "B.Cu") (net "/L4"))
 (segment (start 75.5 68.5) (end 78.54 71.54) (width 0.2) (layer "B.Cu") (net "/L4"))
 (segment (start 78.54 71.54) (end 78.54 73.88) (width 0.2) (layer "B.Cu") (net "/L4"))
 (segment (start 62 68.5) (end 75.5 68.5) (width 0.2) (layer "B.Cu") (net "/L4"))
 (segment (start 60.5 93.23) (end 60.5 70) (width 0.2) (layer "B.Cu") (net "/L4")))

